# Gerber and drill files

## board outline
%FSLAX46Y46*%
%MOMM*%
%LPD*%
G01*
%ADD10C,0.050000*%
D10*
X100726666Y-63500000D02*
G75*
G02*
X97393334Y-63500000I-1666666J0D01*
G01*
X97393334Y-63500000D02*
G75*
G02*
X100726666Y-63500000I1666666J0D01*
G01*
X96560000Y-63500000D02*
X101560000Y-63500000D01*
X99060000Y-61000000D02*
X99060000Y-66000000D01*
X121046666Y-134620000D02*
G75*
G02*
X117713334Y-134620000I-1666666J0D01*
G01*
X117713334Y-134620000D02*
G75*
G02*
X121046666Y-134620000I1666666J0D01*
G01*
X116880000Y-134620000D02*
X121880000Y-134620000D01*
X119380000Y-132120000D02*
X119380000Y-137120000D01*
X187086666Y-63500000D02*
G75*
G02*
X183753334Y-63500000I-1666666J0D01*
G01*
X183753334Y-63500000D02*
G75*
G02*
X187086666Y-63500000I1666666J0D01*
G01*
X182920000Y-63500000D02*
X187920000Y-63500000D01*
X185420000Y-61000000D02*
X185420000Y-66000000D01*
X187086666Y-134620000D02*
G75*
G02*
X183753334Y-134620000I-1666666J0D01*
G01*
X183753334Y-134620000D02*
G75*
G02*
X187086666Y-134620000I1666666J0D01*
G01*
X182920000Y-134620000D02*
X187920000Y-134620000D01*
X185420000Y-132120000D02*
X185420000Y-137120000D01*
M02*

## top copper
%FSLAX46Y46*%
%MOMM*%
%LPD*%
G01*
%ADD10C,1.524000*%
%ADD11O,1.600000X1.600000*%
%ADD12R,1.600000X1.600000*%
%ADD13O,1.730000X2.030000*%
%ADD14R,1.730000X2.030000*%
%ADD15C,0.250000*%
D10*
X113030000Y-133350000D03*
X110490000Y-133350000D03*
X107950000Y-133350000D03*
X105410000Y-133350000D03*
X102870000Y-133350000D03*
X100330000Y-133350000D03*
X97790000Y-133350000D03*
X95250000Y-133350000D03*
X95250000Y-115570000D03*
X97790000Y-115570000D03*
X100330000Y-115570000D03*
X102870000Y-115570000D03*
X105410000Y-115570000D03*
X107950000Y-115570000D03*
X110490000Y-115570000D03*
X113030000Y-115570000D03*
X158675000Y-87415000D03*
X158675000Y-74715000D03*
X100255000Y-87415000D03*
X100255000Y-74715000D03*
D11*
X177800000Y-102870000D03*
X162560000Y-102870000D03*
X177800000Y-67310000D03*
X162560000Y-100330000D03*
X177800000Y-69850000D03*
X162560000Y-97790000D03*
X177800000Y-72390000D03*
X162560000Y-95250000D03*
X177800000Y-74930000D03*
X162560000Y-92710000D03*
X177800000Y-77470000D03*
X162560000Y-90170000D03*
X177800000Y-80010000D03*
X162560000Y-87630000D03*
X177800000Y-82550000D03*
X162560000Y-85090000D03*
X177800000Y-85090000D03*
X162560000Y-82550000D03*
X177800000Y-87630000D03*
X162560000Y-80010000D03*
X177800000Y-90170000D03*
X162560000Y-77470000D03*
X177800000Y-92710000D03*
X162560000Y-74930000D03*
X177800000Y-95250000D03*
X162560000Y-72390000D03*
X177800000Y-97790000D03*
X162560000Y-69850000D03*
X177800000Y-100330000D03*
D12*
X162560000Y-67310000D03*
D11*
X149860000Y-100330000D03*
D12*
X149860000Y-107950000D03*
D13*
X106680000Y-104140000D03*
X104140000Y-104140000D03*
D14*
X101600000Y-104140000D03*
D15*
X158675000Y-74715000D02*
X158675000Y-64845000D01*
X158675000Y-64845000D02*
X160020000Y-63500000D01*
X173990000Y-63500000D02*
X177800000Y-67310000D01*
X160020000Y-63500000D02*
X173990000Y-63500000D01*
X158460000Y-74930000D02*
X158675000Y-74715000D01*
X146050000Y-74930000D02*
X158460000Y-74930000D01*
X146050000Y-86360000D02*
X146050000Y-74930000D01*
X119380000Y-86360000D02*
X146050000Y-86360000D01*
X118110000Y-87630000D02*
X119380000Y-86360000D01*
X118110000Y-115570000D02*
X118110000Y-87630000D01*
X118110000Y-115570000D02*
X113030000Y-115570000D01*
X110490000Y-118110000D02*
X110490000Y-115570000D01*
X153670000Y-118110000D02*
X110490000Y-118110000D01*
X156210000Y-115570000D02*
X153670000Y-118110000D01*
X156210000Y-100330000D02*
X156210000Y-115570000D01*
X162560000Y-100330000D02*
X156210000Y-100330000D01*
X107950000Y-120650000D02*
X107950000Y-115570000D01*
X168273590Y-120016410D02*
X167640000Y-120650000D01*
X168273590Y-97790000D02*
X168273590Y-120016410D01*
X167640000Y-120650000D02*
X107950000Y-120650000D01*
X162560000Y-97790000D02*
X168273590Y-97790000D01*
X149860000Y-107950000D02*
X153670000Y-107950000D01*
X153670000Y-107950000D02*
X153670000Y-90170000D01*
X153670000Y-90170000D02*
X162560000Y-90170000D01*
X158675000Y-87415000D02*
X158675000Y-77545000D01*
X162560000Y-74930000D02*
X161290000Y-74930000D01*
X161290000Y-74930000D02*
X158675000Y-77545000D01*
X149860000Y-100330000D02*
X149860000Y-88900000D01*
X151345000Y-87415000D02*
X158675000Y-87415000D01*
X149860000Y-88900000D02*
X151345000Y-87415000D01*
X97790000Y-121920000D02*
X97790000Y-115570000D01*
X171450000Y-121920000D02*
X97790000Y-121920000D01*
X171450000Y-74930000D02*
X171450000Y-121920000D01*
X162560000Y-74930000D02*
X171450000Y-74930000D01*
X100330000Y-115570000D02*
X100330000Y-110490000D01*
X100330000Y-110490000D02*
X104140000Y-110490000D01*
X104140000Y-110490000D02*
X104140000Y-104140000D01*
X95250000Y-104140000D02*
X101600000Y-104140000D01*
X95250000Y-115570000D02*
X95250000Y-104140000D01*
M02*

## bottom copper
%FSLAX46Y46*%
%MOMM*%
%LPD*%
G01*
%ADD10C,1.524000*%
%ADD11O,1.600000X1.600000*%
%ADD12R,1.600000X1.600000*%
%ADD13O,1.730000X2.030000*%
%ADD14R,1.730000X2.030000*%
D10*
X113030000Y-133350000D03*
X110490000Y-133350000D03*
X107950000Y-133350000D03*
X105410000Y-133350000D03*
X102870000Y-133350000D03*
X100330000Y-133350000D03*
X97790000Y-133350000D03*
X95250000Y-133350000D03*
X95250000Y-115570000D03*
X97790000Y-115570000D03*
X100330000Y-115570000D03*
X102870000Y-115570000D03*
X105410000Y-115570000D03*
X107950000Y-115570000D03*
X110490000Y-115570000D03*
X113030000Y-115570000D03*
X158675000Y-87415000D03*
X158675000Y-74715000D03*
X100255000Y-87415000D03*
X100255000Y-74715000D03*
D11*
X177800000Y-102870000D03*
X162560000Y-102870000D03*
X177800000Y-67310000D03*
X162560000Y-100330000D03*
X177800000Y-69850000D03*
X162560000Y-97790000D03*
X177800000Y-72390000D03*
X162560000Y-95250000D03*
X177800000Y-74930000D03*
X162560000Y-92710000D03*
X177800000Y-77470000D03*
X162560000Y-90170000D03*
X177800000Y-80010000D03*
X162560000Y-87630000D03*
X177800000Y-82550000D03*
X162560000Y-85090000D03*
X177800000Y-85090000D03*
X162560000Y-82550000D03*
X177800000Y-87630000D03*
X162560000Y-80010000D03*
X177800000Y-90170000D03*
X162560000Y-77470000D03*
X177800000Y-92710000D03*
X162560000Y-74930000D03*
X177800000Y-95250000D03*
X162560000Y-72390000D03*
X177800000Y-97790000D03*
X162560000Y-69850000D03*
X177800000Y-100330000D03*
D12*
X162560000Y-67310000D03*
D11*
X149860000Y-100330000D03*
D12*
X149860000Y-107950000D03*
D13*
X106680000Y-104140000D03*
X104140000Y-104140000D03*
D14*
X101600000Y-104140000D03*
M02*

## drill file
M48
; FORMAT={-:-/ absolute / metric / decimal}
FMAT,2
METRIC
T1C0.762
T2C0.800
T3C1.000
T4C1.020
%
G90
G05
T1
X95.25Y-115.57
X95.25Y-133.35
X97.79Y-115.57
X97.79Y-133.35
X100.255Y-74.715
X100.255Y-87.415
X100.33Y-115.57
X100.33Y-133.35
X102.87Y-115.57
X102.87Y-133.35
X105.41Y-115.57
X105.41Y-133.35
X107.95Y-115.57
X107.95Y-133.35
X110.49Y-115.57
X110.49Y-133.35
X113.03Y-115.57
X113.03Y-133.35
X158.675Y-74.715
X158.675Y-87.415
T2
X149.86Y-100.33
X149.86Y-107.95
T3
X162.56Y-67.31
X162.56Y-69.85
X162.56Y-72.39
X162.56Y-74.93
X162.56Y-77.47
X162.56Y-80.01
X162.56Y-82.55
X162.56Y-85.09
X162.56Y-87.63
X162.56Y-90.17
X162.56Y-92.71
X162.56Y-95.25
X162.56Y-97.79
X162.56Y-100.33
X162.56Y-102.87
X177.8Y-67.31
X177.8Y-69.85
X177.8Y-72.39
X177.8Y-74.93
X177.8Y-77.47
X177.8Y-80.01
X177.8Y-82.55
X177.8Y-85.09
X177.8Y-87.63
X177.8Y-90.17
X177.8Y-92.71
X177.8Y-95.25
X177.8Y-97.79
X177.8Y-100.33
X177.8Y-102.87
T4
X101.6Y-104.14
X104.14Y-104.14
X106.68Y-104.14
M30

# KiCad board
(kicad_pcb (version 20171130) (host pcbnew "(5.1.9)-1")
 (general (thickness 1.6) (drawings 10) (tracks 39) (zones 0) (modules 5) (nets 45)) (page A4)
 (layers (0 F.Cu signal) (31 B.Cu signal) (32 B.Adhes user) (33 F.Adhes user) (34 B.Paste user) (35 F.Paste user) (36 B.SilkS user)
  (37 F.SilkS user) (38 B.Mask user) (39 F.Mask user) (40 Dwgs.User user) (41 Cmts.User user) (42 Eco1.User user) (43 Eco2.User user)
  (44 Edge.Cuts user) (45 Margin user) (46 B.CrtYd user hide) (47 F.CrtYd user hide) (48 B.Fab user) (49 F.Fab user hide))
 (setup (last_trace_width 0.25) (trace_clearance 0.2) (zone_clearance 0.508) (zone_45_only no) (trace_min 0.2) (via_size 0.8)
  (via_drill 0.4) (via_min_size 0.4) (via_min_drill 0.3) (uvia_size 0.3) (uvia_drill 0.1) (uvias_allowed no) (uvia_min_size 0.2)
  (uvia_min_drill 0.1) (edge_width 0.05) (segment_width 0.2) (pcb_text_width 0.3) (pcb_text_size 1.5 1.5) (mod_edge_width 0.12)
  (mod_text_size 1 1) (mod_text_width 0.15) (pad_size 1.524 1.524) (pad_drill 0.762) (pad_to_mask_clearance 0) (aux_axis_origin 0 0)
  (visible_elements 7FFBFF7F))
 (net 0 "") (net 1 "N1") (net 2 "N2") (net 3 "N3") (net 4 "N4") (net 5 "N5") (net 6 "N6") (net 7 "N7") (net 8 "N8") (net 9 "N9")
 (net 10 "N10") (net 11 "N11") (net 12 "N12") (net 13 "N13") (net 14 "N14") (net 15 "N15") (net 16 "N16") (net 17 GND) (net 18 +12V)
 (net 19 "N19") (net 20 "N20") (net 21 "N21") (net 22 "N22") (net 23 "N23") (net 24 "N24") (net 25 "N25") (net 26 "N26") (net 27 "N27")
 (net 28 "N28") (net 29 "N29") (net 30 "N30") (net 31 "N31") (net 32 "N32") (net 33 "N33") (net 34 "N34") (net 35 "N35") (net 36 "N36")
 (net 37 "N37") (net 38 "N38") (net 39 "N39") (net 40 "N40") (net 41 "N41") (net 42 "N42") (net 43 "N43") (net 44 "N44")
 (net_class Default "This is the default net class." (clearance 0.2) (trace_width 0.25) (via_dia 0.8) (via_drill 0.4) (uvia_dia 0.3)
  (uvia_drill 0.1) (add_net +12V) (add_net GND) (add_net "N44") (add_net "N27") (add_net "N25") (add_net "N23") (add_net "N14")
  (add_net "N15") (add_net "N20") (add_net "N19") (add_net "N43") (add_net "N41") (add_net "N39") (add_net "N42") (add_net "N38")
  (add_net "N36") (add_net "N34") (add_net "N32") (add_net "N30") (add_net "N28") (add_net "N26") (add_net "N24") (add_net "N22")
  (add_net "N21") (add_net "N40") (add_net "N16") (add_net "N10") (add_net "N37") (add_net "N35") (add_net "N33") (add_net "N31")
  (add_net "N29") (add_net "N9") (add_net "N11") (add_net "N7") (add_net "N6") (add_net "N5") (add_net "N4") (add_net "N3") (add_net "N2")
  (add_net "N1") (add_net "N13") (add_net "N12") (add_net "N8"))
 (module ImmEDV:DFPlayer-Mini (layer F.Cu) (at 114.3 124.46 270)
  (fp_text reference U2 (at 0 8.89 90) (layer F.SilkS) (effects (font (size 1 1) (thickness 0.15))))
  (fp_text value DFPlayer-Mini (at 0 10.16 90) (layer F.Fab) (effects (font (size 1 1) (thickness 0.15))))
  (pad 16 thru_hole circle (at 8.89 1.27 270) (size 1.524 1.524) (drill 0.762) (layers *.Cu *.Mask) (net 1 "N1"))
  (pad 15 thru_hole circle (at 8.89 3.81 270) (size 1.524 1.524) (drill 0.762) (layers *.Cu *.Mask) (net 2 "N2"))
  (pad 14 thru_hole circle (at 8.89 6.35 270) (size 1.524 1.524) (drill 0.762) (layers *.Cu *.Mask) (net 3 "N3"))
  (pad 13 thru_hole circle (at 8.89 8.89 270) (size 1.524 1.524) (drill 0.762) (layers *.Cu *.Mask) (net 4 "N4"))
  (pad 12 thru_hole circle (at 8.89 11.43 270) (size 1.524 1.524) (drill 0.762) (layers *.Cu *.Mask) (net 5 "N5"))
  (pad 11 thru_hole circle (at 8.89 13.97 270) (size 1.524 1.524) (drill 0.762) (layers *.Cu *.Mask) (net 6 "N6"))
  (pad 10 thru_hole circle (at 8.89 16.51 270) (size 1.524 1.524) (drill 0.762) (layers *.Cu *.Mask) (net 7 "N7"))
  (pad 9 thru_hole circle (at 8.89 19.05 270) (size 1.524 1.524) (drill 0.762) (layers *.Cu *.Mask) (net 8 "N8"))
  (pad 8 thru_hole circle (at -8.89 19.05 270) (size 1.524 1.524) (drill 0.762) (layers *.Cu *.Mask) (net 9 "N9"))
  (pad 7 thru_hole circle (at -8.89 16.51 270) (size 1.524 1.524) (drill 0.762) (layers *.Cu *.Mask) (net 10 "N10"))
  (pad 6 thru_hole circle (at -8.89 13.97 270) (size 1.524 1.524) (drill 0.762) (layers *.Cu *.Mask) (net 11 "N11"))
  (pad 5 thru_hole circle (at -8.89 11.43 270) (size 1.524 1.524) (drill 0.762) (layers *.Cu *.Mask) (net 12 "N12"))
  (pad 4 thru_hole circle (at -8.89 8.89 270) (size 1.524 1.524) (drill 0.762) (layers *.Cu *.Mask) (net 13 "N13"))
  (pad 3 thru_hole circle (at -8.89 6.35 270) (size 1.524 1.524) (drill 0.762) (layers *.Cu *.Mask) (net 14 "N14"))
  (pad 2 thru_hole circle (at -8.89 3.81 270) (size 1.524 1.524) (drill 0.762) (layers *.Cu *.Mask) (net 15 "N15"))
  (pad 1 thru_hole circle (at -8.89 1.27 270) (size 1.524 1.524) (drill 0.762) (layers *.Cu *.Mask) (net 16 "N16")))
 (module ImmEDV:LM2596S (layer F.Cu) (at 126.925 79.795)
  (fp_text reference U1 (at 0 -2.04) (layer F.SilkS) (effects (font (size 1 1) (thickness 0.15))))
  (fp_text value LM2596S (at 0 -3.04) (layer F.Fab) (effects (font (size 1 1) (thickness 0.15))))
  (pad 4 thru_hole circle (at 31.75 7.62) (size 1.524 1.524) (drill 0.762) (layers *.Cu *.Mask) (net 10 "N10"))
  (pad 3 thru_hole circle (at 31.75 -5.08) (size 1.524 1.524) (drill 0.762) (layers *.Cu *.Mask) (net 16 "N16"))
  (pad 2 thru_hole circle (at -26.67 7.62) (size 1.524 1.524) (drill 0.762) (layers *.Cu *.Mask) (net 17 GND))
  (pad 1 thru_hole circle (at -26.67 -5.08) (size 1.524 1.524) (drill 0.762) (layers *.Cu *.Mask) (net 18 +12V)))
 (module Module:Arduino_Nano (layer F.Cu) (at 162.56 67.31)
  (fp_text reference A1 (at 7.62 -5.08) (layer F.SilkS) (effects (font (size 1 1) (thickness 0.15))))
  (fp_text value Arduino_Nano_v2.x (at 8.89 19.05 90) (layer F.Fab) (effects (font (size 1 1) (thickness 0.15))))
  (pad 16 thru_hole oval (at 15.24 35.56) (size 1.6 1.6) (drill 1) (layers *.Cu *.Mask) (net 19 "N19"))
  (pad 15 thru_hole oval (at 0 35.56) (size 1.6 1.6) (drill 1) (layers *.Cu *.Mask) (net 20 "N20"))
  (pad 30 thru_hole oval (at 15.24 0) (size 1.6 1.6) (drill 1) (layers *.Cu *.Mask) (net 16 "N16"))
  (pad 14 thru_hole oval (at 0 33.02) (size 1.6 1.6) (drill 1) (layers *.Cu *.Mask) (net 15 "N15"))
  (pad 29 thru_hole oval (at 15.24 2.54) (size 1.6 1.6) (drill 1) (layers *.Cu *.Mask) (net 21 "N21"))
  (pad 13 thru_hole oval (at 0 30.48) (size 1.6 1.6) (drill 1) (layers *.Cu *.Mask) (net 14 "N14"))
  (pad 28 thru_hole oval (at 15.24 5.08) (size 1.6 1.6) (drill 1) (layers *.Cu *.Mask) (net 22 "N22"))
  (pad 12 thru_hole oval (at 0 27.94) (size 1.6 1.6) (drill 1) (layers *.Cu *.Mask) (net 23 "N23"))
  (pad 27 thru_hole oval (at 15.24 7.62) (size 1.6 1.6) (drill 1) (layers *.Cu *.Mask) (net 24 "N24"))
  (pad 11 thru_hole oval (at 0 25.4) (size 1.6 1.6) (drill 1) (layers *.Cu *.Mask) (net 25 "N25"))
  (pad 26 thru_hole oval (at 15.24 10.16) (size 1.6 1.6) (drill 1) (layers *.Cu *.Mask) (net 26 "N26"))
  (pad 10 thru_hole oval (at 0 22.86) (size 1.6 1.6) (drill 1) (layers *.Cu *.Mask) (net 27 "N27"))
  (pad 25 thru_hole oval (at 15.24 12.7) (size 1.6 1.6) (drill 1) (layers *.Cu *.Mask) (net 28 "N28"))
  (pad 9 thru_hole oval (at 0 20.32) (size 1.6 1.6) (drill 1) (layers *.Cu *.Mask) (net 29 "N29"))
  (pad 24 thru_hole oval (at 15.24 15.24) (size 1.6 1.6) (drill 1) (layers *.Cu *.Mask) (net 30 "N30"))
  (pad 8 thru_hole oval (at 0 17.78) (size 1.6 1.6) (drill 1) (layers *.Cu *.Mask) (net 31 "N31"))
  (pad 23 thru_hole oval (at 15.24 17.78) (size 1.6 1.6) (drill 1) (layers *.Cu *.Mask) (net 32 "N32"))
  (pad 7 thru_hole oval (at 0 15.24) (size 1.6 1.6) (drill 1) (layers *.Cu *.Mask) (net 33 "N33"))
  (pad 22 thru_hole oval (at 15.24 20.32) (size 1.6 1.6) (drill 1) (layers *.Cu *.Mask) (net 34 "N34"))
  (pad 6 thru_hole oval (at 0 12.7) (size 1.6 1.6) (drill 1) (layers *.Cu *.Mask) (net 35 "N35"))
  (pad 21 thru_hole oval (at 15.24 22.86) (size 1.6 1.6) (drill 1) (layers *.Cu *.Mask) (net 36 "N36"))
  (pad 5 thru_hole oval (at 0 10.16) (size 1.6 1.6) (drill 1) (layers *.Cu *.Mask) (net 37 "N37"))
  (pad 20 thru_hole oval (at 15.24 25.4) (size 1.6 1.6) (drill 1) (layers *.Cu *.Mask) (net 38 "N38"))
  (pad 4 thru_hole oval (at 0 7.62) (size 1.6 1.6) (drill 1) (layers *.Cu *.Mask) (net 10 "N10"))
  (pad 19 thru_hole oval (at 15.24 27.94) (size 1.6 1.6) (drill 1) (layers *.Cu *.Mask) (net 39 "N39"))
  (pad 3 thru_hole oval (at 0 5.08) (size 1.6 1.6) (drill 1) (layers *.Cu *.Mask) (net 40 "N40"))
  (pad 18 thru_hole oval (at 15.24 30.48) (size 1.6 1.6) (drill 1) (layers *.Cu *.Mask) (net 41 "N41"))
  (pad 2 thru_hole oval (at 0 2.54) (size 1.6 1.6) (drill 1) (layers *.Cu *.Mask) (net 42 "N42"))
  (pad 17 thru_hole oval (at 15.24 33.02) (size 1.6 1.6) (drill 1) (layers *.Cu *.Mask) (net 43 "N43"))
  (pad 1 thru_hole rect (at 0 0) (size 1.6 1.6) (drill 1) (layers *.Cu *.Mask) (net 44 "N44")))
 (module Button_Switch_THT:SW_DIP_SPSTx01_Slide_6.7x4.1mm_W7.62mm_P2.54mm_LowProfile (layer F.Cu) (at 149.86 107.95 90)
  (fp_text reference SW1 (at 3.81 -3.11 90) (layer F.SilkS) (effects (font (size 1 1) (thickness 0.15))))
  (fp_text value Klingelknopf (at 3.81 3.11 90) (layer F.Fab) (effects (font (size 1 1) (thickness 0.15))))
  (pad 2 thru_hole oval (at 7.62 0 90) (size 1.6 1.6) (drill 0.8) (layers *.Cu *.Mask) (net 10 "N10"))
  (pad 1 thru_hole rect (at 0 0 90) (size 1.6 1.6) (drill 0.8) (layers *.Cu *.Mask) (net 27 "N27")))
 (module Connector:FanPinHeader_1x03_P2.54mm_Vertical (layer F.Cu) (at 101.6 104.14)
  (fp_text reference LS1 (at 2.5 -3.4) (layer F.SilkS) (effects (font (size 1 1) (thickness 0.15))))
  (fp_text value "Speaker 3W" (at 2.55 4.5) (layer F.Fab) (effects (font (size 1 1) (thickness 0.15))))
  (pad 3 thru_hole oval (at 5.08 0 90) (size 2.03 1.73) (drill 1.02) (layers *.Cu *.Mask))
  (pad 2 thru_hole oval (at 2.54 0 90) (size 2.03 1.73) (drill 1.02) (layers *.Cu *.Mask) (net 11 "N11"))
  (pad 1 thru_hole rect (at 0 0 90) (size 2.03 1.73) (drill 1.02) (layers *.Cu *.Mask) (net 9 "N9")))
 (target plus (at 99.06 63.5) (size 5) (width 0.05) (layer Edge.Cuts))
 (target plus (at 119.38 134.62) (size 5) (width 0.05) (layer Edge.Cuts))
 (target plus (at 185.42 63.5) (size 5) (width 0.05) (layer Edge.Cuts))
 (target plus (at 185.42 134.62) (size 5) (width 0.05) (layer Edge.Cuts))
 (segment (start 158.675 74.715) (end 158.675 64.845) (width 0.25) (layer F.Cu) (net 16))
 (segment (start 158.675 64.845) (end 160.02 63.5) (width 0.25) (layer F.Cu) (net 16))
 (segment (start 173.99 63.5) (end 177.8 67.31) (width 0.25) (layer F.Cu) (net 16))
 (segment (start 160.02 63.5) (end 173.99 63.5) (width 0.25) (layer F.Cu) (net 16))
 (segment (start 158.46 74.93) (end 158.675 74.715) (width 0.25) (layer F.Cu) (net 16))
 (segment (start 146.05 74.93) (end 158.46 74.93) (width 0.25) (layer F.Cu) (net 16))
 (segment (start 146.05 86.36) (end 146.05 74.93) (width 0.25) (layer F.Cu) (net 16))
 (segment (start 119.38 86.36) (end 146.05 86.36) (width 0.25) (layer F.Cu) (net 16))
 (segment (start 118.11 87.63) (end 119.38 86.36) (width 0.25) (layer F.Cu) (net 16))
 (segment (start 118.11 115.57) (end 118.11 87.63) (width 0.25) (layer F.Cu) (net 16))
 (segment (start 118.11 115.57) (end 113.03 115.57) (width 0.25) (layer F.Cu) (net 16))
 (segment (start 110.49 118.11) (end 110.49 115.57) (width 0.25) (layer F.Cu) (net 15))
 (segment (start 153.67 118.11) (end 110.49 118.11) (width 0.25) (layer F.Cu) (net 15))
 (segment (start 156.21 115.57) (end 153.67 118.11) (width 0.25) (layer F.Cu) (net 15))
 (segment (start 156.21 100.33) (end 156.21 115.57) (width 0.25) (layer F.Cu) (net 15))
 (segment (start 162.56 100.33) (end 156.21 100.33) (width 0.25) (layer F.Cu) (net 15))
 (segment (start 107.95 120.65) (end 107.95 115.57) (width 0.25) (layer F.Cu) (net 14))
 (segment (start 168.27359 120.01641) (end 167.64 120.65) (width 0.25) (layer F.Cu) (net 14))
 (segment (start 168.27359 97.79) (end 168.27359 120.01641) (width 0.25) (layer F.Cu) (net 14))
 (segment (start 167.64 120.65) (end 107.95 120.65) (width 0.25) (layer F.Cu) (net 14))
 (segment (start 162.56 97.79) (end 168.27359 97.79) (width 0.25) (layer F.Cu) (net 14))
 (segment (start 149.86 107.95) (end 153.67 107.95) (width 0.25) (layer F.Cu) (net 27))
 (segment (start 153.67 107.95) (end 153.67 90.17) (width 0.25) (layer F.Cu) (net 27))
 (segment (start 153.67 90.17) (end 162.56 90.17) (width 0.25) (layer F.Cu) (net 27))
 (segment (start 158.675 87.415) (end 158.675 77.545) (width 0.25) (layer F.Cu) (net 10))
 (segment (start 162.56 74.93) (end 161.29 74.93) (width 0.25) (layer F.Cu) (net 10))
 (segment (start 161.29 74.93) (end 158.675 77.545) (width 0.25) (layer F.Cu) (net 10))
 (segment (start 149.86 100.33) (end 149.86 88.9) (width 0.25) (layer F.Cu) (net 10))
 (segment (start 151.345 87.415) (end 158.675 87.415) (width 0.25) (layer F.Cu) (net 10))
 (segment (start 149.86 88.9) (end 151.345 87.415) (width 0.25) (layer F.Cu) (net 10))
 (segment (start 97.79 121.92) (end 97.79 115.57) (width 0.25) (layer F.Cu) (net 10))
 (segment (start 171.45 121.92) (end 97.79 121.92) (width 0.25) (layer F.Cu) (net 10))
 (segment (start 171.45 74.93) (end 171.45 121.92) (width 0.25) (layer F.Cu) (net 10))
 (segment (start 162.56 74.93) (end 171.45 74.93) (width 0.25) (layer F.Cu) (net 10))
 (segment (start 100.33 115.57) (end 100.33 110.49) (width 0.25) (layer F.Cu) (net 11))
 (segment (start 100.33 110.49) (end 104.14 110.49) (width 0.25) (layer F.Cu) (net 11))
 (segment (start 104.14 110.49) (end 104.14 104.14) (width 0.25) (layer F.Cu) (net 11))
 (segment (start 95.25 104.14) (end 101.6 104.14) (width 0.25) (layer F.Cu) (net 9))
 (segment (start 95.25 115.57) (end 95.25 104.14) (width 0.25) (layer F.Cu) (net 9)))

